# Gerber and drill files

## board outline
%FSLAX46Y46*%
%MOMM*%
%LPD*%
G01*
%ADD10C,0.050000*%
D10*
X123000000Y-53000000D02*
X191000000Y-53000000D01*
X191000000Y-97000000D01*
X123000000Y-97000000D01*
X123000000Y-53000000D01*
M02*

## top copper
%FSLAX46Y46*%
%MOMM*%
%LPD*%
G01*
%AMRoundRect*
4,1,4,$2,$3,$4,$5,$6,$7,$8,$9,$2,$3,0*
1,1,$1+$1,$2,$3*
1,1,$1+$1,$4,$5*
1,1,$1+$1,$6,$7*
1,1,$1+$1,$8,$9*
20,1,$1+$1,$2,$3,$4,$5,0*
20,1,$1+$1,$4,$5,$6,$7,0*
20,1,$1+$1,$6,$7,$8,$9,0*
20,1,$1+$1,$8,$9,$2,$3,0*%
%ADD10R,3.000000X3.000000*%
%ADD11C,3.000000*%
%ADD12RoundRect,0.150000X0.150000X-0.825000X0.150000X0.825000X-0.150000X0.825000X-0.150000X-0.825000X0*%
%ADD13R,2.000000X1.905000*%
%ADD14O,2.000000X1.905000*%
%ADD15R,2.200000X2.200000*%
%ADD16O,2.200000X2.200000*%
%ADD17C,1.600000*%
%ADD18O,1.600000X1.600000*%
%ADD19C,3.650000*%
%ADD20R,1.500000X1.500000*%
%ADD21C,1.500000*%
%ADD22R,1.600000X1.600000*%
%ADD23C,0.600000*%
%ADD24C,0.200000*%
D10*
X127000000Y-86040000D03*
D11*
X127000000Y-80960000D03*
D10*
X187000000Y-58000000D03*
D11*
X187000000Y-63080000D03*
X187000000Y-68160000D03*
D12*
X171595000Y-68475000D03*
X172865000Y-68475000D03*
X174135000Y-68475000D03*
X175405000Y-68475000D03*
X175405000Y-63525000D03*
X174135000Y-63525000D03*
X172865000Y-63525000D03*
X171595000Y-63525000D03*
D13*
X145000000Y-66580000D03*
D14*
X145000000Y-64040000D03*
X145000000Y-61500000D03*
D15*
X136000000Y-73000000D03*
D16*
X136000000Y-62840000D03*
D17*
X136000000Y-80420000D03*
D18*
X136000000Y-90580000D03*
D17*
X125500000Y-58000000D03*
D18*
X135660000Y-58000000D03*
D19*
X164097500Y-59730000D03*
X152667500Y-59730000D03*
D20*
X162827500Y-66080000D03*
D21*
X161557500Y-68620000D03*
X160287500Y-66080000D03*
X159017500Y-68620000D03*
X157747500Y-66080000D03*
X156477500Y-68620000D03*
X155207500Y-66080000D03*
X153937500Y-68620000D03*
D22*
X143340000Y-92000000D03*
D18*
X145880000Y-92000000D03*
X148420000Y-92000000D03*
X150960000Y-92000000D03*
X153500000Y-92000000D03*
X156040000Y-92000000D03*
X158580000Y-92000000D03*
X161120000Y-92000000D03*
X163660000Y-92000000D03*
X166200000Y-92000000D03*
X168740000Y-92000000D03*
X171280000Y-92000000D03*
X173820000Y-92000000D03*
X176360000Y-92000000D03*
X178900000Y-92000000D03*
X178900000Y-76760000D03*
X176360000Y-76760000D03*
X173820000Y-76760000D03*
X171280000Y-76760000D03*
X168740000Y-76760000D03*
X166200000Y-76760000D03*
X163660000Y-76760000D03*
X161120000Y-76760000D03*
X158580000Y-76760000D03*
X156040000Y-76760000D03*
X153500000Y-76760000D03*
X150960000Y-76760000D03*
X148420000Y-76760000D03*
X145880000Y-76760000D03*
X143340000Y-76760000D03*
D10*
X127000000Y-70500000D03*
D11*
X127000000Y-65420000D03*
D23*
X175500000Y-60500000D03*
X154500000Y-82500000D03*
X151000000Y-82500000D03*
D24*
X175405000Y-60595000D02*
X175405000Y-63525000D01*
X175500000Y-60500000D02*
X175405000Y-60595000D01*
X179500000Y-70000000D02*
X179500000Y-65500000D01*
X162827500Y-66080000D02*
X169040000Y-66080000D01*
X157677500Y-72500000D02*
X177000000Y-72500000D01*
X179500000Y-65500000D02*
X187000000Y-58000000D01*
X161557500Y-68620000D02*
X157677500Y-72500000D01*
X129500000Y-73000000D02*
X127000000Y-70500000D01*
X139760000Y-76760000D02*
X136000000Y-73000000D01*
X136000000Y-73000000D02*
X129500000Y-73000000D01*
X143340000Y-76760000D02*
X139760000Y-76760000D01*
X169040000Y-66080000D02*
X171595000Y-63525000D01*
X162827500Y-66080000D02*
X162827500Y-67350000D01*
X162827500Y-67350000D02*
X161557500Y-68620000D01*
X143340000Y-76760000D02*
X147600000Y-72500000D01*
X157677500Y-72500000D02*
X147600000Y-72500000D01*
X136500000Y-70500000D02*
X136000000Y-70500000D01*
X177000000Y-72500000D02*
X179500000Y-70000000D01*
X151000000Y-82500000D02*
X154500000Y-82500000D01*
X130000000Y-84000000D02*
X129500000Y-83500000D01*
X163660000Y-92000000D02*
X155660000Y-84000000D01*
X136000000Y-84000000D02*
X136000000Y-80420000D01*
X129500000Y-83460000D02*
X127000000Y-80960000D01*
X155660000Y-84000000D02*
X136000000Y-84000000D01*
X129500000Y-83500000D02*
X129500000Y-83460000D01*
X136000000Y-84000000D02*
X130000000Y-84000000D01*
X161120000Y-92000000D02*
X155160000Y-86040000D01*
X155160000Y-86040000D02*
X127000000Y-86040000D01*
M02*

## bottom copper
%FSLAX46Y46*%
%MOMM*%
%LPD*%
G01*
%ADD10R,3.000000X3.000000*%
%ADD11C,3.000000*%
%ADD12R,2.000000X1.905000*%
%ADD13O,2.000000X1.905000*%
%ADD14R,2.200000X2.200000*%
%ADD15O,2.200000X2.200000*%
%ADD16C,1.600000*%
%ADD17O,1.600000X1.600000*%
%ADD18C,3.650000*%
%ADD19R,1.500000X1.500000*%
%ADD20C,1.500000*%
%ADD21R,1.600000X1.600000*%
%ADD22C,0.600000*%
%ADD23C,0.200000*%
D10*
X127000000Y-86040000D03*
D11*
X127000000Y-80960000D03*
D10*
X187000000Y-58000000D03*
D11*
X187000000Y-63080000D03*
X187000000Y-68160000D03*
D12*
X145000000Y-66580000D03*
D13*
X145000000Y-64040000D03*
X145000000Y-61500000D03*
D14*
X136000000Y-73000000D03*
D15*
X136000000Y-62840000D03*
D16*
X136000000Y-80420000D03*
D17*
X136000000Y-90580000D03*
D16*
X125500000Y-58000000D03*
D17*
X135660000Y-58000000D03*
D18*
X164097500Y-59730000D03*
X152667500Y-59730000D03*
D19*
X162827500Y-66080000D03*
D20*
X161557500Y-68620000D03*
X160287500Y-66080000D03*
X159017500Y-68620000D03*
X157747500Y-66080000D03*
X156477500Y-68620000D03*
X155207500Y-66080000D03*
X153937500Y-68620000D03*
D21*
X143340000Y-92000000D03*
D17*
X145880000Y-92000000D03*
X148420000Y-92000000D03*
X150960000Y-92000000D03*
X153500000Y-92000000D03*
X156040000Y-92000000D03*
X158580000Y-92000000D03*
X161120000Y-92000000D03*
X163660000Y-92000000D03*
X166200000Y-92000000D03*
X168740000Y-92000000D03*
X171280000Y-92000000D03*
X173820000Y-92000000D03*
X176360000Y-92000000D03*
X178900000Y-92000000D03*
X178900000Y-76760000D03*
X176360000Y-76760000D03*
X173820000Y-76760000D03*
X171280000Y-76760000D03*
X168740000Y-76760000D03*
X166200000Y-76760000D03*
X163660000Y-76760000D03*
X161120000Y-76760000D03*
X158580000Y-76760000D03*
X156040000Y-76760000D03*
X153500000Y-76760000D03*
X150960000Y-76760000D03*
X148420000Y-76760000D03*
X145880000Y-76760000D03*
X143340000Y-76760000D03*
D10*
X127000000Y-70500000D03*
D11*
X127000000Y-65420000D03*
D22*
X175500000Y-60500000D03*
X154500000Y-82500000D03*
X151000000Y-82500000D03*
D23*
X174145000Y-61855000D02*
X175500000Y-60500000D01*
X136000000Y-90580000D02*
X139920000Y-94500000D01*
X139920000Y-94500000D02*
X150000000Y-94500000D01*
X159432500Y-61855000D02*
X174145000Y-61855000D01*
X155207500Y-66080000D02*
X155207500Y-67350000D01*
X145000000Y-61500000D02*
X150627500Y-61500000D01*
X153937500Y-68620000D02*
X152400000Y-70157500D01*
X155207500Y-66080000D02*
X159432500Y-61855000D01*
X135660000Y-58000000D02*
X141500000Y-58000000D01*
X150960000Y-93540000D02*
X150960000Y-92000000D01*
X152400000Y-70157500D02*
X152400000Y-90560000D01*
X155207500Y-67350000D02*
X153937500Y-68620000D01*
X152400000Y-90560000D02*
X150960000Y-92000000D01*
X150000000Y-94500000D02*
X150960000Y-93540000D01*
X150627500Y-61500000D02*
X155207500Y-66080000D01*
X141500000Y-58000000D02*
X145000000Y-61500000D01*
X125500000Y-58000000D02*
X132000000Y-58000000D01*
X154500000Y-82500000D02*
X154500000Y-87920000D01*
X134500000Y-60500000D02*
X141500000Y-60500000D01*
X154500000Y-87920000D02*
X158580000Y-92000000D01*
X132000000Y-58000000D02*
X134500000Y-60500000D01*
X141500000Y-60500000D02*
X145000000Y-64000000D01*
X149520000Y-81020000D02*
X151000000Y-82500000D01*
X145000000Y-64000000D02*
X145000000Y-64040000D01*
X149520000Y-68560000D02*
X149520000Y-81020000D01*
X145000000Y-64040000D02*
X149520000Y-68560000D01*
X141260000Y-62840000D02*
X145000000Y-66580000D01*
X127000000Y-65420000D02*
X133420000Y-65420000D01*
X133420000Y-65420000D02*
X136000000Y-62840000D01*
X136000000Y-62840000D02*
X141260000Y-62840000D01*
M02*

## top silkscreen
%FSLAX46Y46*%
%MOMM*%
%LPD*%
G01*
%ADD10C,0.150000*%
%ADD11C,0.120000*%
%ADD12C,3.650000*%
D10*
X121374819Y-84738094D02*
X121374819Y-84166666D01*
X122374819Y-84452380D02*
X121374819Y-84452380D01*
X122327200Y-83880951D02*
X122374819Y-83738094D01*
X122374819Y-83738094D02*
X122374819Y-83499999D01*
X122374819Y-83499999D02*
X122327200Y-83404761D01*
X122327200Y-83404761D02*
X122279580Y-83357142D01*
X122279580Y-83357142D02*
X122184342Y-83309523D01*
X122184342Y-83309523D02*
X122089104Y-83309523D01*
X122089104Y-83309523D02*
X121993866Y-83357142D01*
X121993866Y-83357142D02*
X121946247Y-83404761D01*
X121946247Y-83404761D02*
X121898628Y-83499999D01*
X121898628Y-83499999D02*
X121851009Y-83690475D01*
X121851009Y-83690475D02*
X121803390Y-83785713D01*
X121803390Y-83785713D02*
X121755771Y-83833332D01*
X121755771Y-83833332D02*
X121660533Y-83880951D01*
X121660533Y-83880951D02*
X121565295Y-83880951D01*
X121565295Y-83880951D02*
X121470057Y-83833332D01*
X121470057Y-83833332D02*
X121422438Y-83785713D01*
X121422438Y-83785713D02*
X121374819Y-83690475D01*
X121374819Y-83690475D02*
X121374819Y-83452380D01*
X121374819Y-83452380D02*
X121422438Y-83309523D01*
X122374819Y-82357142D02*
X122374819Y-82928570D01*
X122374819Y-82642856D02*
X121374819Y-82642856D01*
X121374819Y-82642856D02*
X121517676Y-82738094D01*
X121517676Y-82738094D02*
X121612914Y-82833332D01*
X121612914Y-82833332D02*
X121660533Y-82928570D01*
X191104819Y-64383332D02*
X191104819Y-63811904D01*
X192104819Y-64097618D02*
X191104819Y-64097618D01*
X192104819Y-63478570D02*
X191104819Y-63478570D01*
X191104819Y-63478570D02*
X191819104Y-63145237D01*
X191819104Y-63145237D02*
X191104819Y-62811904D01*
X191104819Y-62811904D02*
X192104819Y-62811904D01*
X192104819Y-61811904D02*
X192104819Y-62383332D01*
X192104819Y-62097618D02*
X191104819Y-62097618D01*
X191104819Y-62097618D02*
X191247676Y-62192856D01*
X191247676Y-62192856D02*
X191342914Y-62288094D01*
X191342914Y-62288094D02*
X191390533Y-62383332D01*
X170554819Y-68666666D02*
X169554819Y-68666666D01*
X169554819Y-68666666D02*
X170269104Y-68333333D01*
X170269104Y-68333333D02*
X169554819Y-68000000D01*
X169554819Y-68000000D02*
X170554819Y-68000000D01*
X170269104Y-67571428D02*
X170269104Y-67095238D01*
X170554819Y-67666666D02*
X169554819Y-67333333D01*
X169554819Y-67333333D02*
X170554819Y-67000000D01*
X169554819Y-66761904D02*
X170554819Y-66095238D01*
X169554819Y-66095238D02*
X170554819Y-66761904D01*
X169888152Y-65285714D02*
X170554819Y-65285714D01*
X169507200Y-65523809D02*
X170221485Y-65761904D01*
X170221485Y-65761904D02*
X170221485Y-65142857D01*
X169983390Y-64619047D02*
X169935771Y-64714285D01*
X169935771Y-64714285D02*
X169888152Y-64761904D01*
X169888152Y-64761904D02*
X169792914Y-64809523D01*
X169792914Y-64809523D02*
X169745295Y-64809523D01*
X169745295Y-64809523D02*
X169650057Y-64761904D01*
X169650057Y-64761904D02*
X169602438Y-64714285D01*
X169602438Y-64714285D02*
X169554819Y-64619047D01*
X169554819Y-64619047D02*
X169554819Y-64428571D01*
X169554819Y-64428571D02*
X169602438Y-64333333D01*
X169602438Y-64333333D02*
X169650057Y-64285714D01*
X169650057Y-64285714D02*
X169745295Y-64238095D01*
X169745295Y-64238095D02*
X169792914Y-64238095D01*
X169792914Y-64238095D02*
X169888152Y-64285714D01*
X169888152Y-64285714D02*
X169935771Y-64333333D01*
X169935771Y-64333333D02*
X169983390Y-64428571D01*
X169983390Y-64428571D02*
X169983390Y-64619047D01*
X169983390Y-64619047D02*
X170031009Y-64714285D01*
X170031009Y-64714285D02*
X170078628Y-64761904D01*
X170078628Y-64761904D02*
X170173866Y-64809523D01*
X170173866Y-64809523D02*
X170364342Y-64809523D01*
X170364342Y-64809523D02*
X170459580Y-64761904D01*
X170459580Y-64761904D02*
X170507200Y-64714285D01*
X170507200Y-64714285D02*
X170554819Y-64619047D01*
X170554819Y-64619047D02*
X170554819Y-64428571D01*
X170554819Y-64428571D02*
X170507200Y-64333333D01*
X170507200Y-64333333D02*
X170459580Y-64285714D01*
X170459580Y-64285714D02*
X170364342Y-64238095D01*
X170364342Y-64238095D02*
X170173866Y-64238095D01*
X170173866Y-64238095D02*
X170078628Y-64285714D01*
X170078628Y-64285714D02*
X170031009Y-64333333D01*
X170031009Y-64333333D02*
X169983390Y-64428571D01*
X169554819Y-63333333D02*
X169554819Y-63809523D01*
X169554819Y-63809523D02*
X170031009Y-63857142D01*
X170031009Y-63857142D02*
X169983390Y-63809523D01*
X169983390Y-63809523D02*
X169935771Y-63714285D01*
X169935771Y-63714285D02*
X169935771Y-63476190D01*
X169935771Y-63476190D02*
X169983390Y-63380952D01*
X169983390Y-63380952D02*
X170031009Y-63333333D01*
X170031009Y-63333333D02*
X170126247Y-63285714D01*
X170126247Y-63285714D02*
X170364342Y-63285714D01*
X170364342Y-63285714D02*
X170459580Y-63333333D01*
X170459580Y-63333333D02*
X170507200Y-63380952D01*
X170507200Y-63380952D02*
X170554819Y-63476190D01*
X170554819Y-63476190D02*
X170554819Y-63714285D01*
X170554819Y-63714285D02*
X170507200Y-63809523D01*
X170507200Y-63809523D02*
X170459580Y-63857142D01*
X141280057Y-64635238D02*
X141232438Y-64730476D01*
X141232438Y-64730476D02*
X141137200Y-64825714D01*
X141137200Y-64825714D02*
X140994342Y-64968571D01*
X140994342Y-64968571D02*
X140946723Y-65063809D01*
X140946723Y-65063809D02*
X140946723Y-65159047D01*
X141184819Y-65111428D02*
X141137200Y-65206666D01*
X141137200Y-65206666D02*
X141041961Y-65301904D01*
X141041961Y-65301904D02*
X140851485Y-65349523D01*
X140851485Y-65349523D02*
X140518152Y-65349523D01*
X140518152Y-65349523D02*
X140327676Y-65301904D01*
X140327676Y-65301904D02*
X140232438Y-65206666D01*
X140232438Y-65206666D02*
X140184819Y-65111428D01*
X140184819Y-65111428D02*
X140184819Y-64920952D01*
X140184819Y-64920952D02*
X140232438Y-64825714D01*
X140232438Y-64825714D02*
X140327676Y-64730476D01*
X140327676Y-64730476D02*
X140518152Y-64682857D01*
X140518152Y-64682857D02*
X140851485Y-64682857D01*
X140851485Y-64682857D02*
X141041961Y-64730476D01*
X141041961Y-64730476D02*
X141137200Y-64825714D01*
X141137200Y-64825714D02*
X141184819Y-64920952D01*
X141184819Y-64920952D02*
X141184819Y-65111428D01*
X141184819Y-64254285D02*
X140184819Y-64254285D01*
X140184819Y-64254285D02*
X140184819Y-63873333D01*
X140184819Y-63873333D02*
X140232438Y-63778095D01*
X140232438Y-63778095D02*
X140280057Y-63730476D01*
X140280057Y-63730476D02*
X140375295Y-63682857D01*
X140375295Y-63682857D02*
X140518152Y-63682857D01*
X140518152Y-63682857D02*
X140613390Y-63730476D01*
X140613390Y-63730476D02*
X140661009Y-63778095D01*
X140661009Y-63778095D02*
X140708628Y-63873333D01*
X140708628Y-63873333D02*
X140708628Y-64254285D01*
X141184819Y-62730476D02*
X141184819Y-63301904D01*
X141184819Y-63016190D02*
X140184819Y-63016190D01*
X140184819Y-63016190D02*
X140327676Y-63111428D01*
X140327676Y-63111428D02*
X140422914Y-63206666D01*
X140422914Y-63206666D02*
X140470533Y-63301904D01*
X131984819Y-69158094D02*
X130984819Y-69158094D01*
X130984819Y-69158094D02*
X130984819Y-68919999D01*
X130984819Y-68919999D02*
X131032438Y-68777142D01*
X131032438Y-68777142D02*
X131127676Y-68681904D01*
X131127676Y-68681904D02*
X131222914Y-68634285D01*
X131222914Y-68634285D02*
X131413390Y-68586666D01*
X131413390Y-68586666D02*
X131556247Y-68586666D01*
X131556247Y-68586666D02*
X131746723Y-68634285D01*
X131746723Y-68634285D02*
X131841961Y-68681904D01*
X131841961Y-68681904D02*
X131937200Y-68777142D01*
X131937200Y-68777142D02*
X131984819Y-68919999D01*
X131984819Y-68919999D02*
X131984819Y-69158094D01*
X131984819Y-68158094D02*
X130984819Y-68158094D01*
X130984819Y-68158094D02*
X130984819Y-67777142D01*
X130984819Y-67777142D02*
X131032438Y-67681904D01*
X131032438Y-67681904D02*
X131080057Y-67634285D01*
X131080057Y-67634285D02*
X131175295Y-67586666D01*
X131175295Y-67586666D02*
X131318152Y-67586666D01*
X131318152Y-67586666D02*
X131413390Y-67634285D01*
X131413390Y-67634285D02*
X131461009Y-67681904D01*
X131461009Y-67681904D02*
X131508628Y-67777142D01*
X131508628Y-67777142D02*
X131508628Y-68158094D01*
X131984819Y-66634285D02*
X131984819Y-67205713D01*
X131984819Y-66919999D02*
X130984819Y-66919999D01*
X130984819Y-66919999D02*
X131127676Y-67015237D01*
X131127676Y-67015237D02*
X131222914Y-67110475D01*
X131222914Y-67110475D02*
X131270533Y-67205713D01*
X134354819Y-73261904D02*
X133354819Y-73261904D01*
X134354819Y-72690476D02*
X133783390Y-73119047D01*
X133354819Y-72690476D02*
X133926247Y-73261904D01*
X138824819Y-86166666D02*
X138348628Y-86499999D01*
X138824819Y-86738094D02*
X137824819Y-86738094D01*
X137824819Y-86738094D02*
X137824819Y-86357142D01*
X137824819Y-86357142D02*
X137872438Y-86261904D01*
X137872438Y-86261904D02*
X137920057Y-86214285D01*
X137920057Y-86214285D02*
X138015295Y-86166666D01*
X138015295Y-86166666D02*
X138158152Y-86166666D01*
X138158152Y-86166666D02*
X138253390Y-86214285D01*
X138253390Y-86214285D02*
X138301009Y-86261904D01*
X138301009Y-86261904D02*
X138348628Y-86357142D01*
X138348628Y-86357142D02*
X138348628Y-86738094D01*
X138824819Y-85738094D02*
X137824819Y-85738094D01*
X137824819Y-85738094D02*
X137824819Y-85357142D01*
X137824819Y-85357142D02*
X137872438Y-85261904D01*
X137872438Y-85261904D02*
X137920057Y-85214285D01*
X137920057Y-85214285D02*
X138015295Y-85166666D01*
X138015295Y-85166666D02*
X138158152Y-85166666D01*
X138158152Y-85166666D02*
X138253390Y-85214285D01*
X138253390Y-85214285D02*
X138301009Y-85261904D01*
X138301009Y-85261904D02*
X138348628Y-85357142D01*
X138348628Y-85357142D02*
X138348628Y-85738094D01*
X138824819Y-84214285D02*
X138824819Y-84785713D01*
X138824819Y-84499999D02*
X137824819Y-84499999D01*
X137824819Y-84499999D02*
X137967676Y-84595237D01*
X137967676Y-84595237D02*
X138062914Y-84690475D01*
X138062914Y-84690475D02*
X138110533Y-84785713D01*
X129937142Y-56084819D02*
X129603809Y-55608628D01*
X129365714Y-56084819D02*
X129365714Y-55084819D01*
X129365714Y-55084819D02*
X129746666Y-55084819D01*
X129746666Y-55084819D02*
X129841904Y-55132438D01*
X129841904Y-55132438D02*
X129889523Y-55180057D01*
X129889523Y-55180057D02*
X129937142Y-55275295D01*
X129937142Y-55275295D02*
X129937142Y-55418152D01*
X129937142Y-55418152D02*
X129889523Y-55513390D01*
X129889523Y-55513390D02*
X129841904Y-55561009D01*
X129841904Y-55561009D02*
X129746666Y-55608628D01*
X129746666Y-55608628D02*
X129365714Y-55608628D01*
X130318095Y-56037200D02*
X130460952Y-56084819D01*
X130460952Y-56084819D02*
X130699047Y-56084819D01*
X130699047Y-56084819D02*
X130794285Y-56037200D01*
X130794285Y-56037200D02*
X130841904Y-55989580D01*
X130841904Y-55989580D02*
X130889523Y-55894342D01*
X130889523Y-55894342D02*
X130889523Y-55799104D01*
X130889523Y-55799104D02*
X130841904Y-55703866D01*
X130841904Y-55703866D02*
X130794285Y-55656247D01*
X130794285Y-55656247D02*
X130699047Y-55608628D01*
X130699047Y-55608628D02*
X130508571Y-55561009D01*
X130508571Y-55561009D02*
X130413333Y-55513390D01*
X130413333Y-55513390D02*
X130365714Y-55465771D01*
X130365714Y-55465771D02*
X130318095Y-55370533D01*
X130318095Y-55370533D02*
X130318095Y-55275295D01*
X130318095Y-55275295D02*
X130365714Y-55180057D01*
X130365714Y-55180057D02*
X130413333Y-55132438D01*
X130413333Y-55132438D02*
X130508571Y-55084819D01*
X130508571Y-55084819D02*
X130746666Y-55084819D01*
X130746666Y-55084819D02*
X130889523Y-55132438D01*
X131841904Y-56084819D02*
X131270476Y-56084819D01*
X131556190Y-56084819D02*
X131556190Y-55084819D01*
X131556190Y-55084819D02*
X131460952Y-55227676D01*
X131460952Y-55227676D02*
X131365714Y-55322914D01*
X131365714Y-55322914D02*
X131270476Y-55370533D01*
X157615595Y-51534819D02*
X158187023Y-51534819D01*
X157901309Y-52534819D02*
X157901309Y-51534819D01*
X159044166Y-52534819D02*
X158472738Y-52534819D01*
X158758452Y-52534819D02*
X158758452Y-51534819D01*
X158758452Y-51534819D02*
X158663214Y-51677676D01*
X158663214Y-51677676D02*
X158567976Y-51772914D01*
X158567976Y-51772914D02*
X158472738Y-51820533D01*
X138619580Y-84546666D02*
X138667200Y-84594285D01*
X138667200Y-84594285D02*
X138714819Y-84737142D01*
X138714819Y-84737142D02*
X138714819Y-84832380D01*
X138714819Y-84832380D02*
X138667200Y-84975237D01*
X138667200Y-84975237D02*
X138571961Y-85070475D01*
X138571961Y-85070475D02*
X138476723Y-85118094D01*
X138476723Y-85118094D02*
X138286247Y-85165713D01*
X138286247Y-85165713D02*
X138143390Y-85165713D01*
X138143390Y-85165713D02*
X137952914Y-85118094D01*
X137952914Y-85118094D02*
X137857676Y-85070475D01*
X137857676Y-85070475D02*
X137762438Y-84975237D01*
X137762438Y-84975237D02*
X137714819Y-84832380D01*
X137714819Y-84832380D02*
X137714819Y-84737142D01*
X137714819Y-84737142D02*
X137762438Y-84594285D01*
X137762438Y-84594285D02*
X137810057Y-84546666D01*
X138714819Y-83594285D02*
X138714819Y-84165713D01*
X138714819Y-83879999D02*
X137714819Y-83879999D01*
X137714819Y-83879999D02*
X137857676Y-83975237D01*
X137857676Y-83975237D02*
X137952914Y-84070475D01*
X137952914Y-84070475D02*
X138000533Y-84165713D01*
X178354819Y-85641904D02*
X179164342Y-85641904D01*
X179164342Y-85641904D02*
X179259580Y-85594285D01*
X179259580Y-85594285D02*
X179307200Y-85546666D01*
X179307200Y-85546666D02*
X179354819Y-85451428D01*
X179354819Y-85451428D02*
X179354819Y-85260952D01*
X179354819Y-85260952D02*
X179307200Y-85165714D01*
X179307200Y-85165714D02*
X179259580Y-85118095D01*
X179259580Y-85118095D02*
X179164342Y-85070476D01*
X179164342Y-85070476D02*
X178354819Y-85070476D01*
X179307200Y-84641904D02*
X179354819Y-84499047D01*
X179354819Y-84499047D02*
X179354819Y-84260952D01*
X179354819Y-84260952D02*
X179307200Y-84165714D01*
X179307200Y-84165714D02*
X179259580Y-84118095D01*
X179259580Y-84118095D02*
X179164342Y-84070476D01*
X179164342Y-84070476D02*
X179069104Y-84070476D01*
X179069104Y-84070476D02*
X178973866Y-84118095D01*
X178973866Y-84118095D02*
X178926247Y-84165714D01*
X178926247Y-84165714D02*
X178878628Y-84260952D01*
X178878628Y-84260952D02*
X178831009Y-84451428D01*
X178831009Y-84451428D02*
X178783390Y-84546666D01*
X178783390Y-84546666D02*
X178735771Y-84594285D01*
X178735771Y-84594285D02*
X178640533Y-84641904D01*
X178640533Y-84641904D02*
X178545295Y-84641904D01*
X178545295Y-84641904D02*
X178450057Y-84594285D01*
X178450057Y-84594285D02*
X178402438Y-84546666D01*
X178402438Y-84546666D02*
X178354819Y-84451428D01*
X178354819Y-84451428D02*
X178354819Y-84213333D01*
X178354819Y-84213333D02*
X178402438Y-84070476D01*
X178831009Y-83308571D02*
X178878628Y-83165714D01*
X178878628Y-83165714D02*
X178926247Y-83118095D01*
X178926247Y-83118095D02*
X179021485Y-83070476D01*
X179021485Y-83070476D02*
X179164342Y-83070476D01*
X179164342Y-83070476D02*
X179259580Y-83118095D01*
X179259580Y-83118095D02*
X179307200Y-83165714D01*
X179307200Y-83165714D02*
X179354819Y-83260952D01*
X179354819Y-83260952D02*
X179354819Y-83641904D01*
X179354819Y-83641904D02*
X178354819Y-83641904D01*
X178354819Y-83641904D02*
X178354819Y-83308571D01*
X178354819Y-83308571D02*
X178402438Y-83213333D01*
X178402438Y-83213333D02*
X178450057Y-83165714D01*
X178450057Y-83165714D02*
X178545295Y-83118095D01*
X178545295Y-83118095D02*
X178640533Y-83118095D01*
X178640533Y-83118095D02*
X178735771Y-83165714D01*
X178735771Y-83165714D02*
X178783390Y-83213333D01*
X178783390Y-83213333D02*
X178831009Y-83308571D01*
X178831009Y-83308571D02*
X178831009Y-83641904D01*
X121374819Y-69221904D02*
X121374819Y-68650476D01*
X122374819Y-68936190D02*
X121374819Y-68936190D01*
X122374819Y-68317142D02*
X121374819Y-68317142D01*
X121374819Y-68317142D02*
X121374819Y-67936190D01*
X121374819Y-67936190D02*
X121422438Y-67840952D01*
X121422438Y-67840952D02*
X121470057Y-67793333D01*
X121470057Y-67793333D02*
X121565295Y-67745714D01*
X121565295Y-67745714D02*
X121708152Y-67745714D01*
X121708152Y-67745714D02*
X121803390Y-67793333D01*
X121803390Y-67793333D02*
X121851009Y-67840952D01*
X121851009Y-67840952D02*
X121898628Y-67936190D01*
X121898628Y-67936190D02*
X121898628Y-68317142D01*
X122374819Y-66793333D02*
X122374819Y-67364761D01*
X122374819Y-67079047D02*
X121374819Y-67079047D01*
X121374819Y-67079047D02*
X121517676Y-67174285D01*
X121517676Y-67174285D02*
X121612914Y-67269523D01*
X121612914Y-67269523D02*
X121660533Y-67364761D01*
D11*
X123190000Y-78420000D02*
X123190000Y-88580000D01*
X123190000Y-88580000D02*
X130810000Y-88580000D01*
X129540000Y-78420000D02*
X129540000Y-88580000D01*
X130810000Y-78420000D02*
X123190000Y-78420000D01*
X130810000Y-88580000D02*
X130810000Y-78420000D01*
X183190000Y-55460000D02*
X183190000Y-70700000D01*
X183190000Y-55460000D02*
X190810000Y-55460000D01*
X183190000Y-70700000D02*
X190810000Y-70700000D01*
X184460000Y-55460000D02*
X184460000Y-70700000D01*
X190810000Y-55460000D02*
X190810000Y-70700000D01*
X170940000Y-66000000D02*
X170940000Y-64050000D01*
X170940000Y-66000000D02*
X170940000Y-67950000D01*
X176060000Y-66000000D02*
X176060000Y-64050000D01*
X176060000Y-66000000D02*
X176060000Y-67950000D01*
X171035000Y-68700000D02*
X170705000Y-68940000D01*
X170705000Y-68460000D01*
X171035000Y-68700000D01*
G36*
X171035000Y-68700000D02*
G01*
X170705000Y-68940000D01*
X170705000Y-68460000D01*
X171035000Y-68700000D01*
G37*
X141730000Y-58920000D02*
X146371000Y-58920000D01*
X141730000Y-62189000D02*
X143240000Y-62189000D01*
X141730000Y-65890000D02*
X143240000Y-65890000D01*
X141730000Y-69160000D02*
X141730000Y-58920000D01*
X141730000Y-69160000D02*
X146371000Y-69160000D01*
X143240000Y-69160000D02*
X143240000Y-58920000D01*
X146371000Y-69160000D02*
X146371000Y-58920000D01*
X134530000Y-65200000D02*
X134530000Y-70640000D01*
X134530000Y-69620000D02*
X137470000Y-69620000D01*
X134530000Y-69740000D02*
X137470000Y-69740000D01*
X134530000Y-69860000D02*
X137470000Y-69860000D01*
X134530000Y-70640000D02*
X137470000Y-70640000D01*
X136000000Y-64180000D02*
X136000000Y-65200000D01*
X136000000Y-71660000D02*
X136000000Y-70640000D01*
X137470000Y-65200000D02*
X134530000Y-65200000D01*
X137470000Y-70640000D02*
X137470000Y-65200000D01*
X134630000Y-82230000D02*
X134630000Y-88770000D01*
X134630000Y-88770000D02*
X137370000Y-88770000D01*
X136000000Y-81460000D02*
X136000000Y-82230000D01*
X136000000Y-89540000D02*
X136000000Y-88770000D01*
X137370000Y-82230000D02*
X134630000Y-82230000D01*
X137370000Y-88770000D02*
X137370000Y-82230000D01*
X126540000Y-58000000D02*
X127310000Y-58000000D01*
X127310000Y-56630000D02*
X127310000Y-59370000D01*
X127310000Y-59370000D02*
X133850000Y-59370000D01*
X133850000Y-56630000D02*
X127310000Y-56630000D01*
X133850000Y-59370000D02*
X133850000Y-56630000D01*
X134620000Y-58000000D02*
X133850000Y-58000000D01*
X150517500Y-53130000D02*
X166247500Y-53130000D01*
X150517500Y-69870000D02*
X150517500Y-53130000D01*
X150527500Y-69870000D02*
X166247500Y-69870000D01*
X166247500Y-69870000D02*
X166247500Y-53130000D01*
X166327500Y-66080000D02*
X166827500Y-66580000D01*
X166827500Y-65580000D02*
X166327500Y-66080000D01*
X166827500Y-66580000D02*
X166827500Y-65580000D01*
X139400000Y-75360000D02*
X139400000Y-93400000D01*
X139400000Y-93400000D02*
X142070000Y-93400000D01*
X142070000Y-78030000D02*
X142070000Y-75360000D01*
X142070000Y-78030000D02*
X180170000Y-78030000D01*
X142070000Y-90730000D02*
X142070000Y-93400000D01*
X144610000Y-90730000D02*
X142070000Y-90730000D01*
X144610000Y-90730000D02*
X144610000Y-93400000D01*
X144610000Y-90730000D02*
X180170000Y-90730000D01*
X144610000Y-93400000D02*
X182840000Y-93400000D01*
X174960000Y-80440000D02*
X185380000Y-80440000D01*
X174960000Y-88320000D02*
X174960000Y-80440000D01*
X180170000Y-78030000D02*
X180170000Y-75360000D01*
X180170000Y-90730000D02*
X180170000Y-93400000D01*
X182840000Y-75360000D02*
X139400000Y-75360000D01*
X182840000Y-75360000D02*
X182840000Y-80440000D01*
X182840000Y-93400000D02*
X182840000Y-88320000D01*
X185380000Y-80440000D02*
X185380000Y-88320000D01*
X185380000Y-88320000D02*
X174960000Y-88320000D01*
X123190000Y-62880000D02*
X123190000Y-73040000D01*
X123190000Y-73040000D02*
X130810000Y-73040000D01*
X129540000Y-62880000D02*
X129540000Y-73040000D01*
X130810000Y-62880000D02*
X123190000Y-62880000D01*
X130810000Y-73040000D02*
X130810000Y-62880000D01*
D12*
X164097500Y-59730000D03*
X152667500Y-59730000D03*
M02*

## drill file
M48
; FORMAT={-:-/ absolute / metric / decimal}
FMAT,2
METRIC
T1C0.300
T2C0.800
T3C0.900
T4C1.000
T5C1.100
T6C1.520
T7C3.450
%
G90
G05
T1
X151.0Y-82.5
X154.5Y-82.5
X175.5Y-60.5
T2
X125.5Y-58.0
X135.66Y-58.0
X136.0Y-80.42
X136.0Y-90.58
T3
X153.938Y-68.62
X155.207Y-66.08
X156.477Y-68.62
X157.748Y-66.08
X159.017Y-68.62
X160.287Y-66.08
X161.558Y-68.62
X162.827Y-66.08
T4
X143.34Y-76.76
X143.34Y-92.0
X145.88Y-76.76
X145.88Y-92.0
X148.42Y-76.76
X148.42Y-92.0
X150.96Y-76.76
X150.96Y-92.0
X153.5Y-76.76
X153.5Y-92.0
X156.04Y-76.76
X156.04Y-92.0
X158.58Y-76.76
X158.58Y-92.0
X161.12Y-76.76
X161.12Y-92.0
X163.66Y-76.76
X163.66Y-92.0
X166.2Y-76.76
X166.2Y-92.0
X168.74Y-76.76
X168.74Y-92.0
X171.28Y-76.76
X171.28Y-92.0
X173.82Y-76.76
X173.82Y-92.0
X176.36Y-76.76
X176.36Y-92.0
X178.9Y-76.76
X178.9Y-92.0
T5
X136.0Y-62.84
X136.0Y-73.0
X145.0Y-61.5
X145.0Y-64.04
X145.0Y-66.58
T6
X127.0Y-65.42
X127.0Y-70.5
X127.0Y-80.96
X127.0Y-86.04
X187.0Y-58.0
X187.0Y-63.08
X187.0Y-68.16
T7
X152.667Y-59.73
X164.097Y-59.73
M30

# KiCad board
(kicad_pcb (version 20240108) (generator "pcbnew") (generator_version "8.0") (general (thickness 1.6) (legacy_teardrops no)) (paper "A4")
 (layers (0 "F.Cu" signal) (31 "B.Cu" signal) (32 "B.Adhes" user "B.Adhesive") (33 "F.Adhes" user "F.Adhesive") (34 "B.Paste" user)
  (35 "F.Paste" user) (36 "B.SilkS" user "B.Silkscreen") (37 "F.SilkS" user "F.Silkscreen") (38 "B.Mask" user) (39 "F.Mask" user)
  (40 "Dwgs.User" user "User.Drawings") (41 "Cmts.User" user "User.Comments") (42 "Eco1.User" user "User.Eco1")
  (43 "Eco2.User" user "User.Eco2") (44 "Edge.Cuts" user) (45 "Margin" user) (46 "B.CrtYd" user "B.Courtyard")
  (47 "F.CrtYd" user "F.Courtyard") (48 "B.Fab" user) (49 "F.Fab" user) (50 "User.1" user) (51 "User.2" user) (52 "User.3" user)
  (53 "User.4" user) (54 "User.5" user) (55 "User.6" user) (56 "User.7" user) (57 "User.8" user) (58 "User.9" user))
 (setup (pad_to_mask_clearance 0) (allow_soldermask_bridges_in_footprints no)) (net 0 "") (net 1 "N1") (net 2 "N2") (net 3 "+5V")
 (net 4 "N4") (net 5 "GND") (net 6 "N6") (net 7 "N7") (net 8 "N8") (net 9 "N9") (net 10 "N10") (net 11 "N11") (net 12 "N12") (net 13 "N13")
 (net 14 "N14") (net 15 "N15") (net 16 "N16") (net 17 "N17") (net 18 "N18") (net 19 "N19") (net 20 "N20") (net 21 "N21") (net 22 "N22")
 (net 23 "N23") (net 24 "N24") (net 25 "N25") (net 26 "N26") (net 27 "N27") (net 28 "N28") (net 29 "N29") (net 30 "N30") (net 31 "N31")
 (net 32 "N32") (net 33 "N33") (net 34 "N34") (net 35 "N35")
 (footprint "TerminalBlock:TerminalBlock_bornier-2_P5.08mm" (layer "F.Cu") (at 127 86.04 90)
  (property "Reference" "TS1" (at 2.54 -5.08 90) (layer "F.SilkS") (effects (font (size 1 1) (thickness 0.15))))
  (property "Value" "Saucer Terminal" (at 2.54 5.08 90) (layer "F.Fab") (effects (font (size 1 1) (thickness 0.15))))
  (fp_line (start 7.62 -3.81) (end -2.54 -3.81) (stroke (width 0.12) (type solid)) (layer "F.SilkS"))
  (fp_line (start -2.54 -3.81) (end -2.54 3.81) (stroke (width 0.12) (type solid)) (layer "F.SilkS"))
  (fp_line (start 7.62 2.54) (end -2.54 2.54) (stroke (width 0.12) (type solid)) (layer "F.SilkS"))
  (fp_line (start 7.62 3.81) (end 7.62 -3.81) (stroke (width 0.12) (type solid)) (layer "F.SilkS"))
  (fp_line (start -2.54 3.81) (end 7.62 3.81) (stroke (width 0.12) (type solid)) (layer "F.SilkS"))
  (pad "1" thru_hole rect (at 0 0 90) (size 3 3) (drill 1.52) (layers "*.Cu" "*.Mask") (remove_unused_layers no) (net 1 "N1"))
  (pad "2" thru_hole circle (at 5.08 0 90) (size 3 3) (drill 1.52) (layers "*.Cu" "*.Mask") (remove_unused_layers no) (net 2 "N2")))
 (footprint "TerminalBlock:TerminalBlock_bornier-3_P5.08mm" (layer "F.Cu") (at 187 58 -90)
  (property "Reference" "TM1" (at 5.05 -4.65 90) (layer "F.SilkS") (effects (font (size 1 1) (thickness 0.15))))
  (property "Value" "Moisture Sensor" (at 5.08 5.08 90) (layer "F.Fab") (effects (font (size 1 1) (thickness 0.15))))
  (fp_line (start -2.54 3.81) (end 12.7 3.81) (stroke (width 0.12) (type solid)) (layer "F.SilkS"))
  (fp_line (start -2.54 3.81) (end -2.54 -3.81) (stroke (width 0.12) (type solid)) (layer "F.SilkS"))
  (fp_line (start 12.7 3.81) (end 12.7 -3.81) (stroke (width 0.12) (type solid)) (layer "F.SilkS"))
  (fp_line (start -2.54 2.54) (end 12.7 2.54) (stroke (width 0.12) (type solid)) (layer "F.SilkS"))
  (fp_line (start -2.54 -3.81) (end 12.7 -3.81) (stroke (width 0.12) (type solid)) (layer "F.SilkS"))
  (pad "1" thru_hole rect (at 0 0 270) (size 3 3) (drill 1.52) (layers "*.Cu" "*.Mask") (remove_unused_layers no) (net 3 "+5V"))
  (pad "2" thru_hole circle (at 5.08 0 270) (size 3 3) (drill 1.52) (layers "*.Cu" "*.Mask") (remove_unused_layers no) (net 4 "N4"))
  (pad "3" thru_hole circle (at 10.16 0 270) (size 3 3) (drill 1.52) (layers "*.Cu" "*.Mask") (remove_unused_layers no) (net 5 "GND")))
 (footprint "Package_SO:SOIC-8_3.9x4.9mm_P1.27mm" (layer "F.Cu") (at 173.5 66 90)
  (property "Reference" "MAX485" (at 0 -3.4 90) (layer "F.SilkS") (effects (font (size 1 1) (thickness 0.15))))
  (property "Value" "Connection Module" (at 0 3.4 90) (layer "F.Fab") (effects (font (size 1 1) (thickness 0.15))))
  (fp_line (start 0 -2.56) (end 1.95 -2.56) (stroke (width 0.12) (type solid)) (layer "F.SilkS"))
  (fp_line (start 0 -2.56) (end -1.95 -2.56) (stroke (width 0.12) (type solid)) (layer "F.SilkS"))
  (fp_line (start 0 2.56) (end 1.95 2.56) (stroke (width 0.12) (type solid)) (layer "F.SilkS"))
  (fp_line (start 0 2.56) (end -1.95 2.56) (stroke (width 0.12) (type solid)) (layer "F.SilkS"))
  (fp_poly
   (pts (xy -2.7 -2.465) (xy -2.94 -2.795) (xy -2.46 -2.795) (xy -2.7 -2.465)) (stroke (width 0.12) (type solid)) (fill solid)
   (layer "F.SilkS"))
  (pad "1" smd roundrect (at -2.475 -1.905 90) (size 1.95 0.6) (layers "F.Cu" "F.Paste" "F.Mask") (roundrect_rratio 0.25) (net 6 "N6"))
  (pad "2" smd roundrect (at -2.475 -0.635 90) (size 1.95 0.6) (layers "F.Cu" "F.Paste" "F.Mask") (roundrect_rratio 0.25) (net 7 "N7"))
  (pad "3" smd roundrect (at -2.475 0.635 90) (size 1.95 0.6) (layers "F.Cu" "F.Paste" "F.Mask") (roundrect_rratio 0.25) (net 7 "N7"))
  (pad "4" smd roundrect (at -2.475 1.905 90) (size 1.95 0.6) (layers "F.Cu" "F.Paste" "F.Mask") (roundrect_rratio 0.25) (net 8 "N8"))
  (pad "5" smd roundrect (at 2.475 1.905 90) (size 1.95 0.6) (layers "F.Cu" "F.Paste" "F.Mask") (roundrect_rratio 0.25) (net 5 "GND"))
  (pad "6" smd roundrect (at 2.475 0.635 90) (size 1.95 0.6) (layers "F.Cu" "F.Paste" "F.Mask") (roundrect_rratio 0.25) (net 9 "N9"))
  (pad "7" smd roundrect (at 2.475 -0.635 90) (size 1.95 0.6) (layers "F.Cu" "F.Paste" "F.Mask") (roundrect_rratio 0.25) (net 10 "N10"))
  (pad "8" smd roundrect (at 2.475 -1.905 90) (size 1.95 0.6) (layers "F.Cu" "F.Paste" "F.Mask") (roundrect_rratio 0.25) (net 3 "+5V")))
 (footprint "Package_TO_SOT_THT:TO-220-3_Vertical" (layer "F.Cu") (at 145 66.58 90)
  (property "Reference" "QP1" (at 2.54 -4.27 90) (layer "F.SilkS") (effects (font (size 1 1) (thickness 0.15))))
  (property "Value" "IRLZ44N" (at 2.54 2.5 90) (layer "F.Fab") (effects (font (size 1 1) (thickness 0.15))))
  (fp_line (start 7.66 -3.27) (end 7.66 1.371) (stroke (width 0.12) (type solid)) (layer "F.SilkS"))
  (fp_line (start 4.391 -3.27) (end 4.391 -1.76) (stroke (width 0.12) (type solid)) (layer "F.SilkS"))
  (fp_line (start 0.69 -3.27) (end 0.69 -1.76) (stroke (width 0.12) (type solid)) (layer "F.SilkS"))
  (fp_line (start -2.58 -3.27) (end 7.66 -3.27) (stroke (width 0.12) (type solid)) (layer "F.SilkS"))
  (fp_line (start -2.58 -3.27) (end -2.58 1.371) (stroke (width 0.12) (type solid)) (layer "F.SilkS"))
  (fp_line (start -2.58 -1.76) (end 7.66 -1.76) (stroke (width 0.12) (type solid)) (layer "F.SilkS"))
  (fp_line (start -2.58 1.371) (end 7.66 1.371) (stroke (width 0.12) (type solid)) (layer "F.SilkS"))
  (pad "1" thru_hole rect (at 0 0 90) (size 1.905 2) (drill 1.1) (layers "*.Cu" "*.Mask") (remove_unused_layers no) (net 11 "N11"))
  (pad "2" thru_hole oval (at 2.54 0 90) (size 1.905 2) (drill 1.1) (layers "*.Cu" "*.Mask") (remove_unused_layers no) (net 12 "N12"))
  (pad "3" thru_hole oval (at 5.08 0 90) (size 1.905 2) (drill 1.1) (layers "*.Cu" "*.Mask") (remove_unused_layers no) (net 5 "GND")))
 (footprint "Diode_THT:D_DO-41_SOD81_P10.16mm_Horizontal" (layer "F.Cu") (at 136 73 90)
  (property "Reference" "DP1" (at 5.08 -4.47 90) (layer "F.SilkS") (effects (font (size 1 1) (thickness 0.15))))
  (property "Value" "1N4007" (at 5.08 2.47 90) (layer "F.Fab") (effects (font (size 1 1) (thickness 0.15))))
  (fp_line (start 7.8 -1.47) (end 2.36 -1.47) (stroke (width 0.12) (type solid)) (layer "F.SilkS"))
  (fp_line (start 3.38 -1.47) (end 3.38 1.47) (stroke (width 0.12) (type solid)) (layer "F.SilkS"))
  (fp_line (start 3.26 -1.47) (end 3.26 1.47) (stroke (width 0.12) (type solid)) (layer "F.SilkS"))
  (fp_line (start 3.14 -1.47) (end 3.14 1.47) (stroke (width 0.12) (type solid)) (layer "F.SilkS"))
  (fp_line (start 2.36 -1.47) (end 2.36 1.47) (stroke (width 0.12) (type solid)) (layer "F.SilkS"))
  (fp_line (start 8.82 0) (end 7.8 0) (stroke (width 0.12) (type solid)) (layer "F.SilkS"))
  (fp_line (start 1.34 0) (end 2.36 0) (stroke (width 0.12) (type solid)) (layer "F.SilkS"))
  (fp_line (start 7.8 1.47) (end 7.8 -1.47) (stroke (width 0.12) (type solid)) (layer "F.SilkS"))
  (fp_line (start 2.36 1.47) (end 7.8 1.47) (stroke (width 0.12) (type solid)) (layer "F.SilkS"))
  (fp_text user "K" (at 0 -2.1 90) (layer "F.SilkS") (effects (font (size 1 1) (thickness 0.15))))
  (pad "1" thru_hole rect (at 0 0 90) (size 2.2 2.2) (drill 1.1) (layers "*.Cu" "*.Mask") (remove_unused_layers no) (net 3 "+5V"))
  (pad "2" thru_hole oval (at 10.16 0 90) (size 2.2 2.2) (drill 1.1) (layers "*.Cu" "*.Mask") (remove_unused_layers no) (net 11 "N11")))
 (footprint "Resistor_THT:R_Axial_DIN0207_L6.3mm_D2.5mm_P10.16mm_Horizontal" (layer "F.Cu") (at 136 80.42 -90)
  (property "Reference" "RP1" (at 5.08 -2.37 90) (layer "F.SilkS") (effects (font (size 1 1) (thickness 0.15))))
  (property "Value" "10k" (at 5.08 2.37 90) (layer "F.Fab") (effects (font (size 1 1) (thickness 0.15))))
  (fp_line (start 1.81 1.37) (end 8.35 1.37) (stroke (width 0.12) (type solid)) (layer "F.SilkS"))
  (fp_line (start 8.35 1.37) (end 8.35 -1.37) (stroke (width 0.12) (type solid)) (layer "F.SilkS"))
  (fp_line (start 1.04 0) (end 1.81 0) (stroke (width 0.12) (type solid)) (layer "F.SilkS"))
  (fp_line (start 9.12 0) (end 8.35 0) (stroke (width 0.12) (type solid)) (layer "F.SilkS"))
  (fp_line (start 1.81 -1.37) (end 1.81 1.37) (stroke (width 0.12) (type solid)) (layer "F.SilkS"))
  (fp_line (start 8.35 -1.37) (end 1.81 -1.37) (stroke (width 0.12) (type solid)) (layer "F.SilkS"))
  (pad "1" thru_hole circle (at 0 0 270) (size 1.6 1.6) (drill 0.8) (layers "*.Cu" "*.Mask") (remove_unused_layers no) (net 2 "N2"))
  (pad "2" thru_hole oval (at 10.16 0 270) (size 1.6 1.6) (drill 0.8) (layers "*.Cu" "*.Mask") (remove_unused_layers no) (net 5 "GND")))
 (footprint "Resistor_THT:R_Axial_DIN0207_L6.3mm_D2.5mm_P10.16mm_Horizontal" (layer "F.Cu") (at 125.5 58)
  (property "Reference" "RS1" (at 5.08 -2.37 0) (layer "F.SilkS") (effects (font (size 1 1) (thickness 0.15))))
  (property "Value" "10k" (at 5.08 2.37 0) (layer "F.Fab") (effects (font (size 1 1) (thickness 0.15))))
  (fp_line (start 1.04 0) (end 1.81 0) (stroke (width 0.12) (type solid)) (layer "F.SilkS"))
  (fp_line (start 1.81 -1.37) (end 1.81 1.37) (stroke (width 0.12) (type solid)) (layer "F.SilkS"))
  (fp_line (start 1.81 1.37) (end 8.35 1.37) (stroke (width 0.12) (type solid)) (layer "F.SilkS"))
  (fp_line (start 8.35 -1.37) (end 1.81 -1.37) (stroke (width 0.12) (type solid)) (layer "F.SilkS"))
  (fp_line (start 8.35 1.37) (end 8.35 -1.37) (stroke (width 0.12) (type solid)) (layer "F.SilkS"))
  (fp_line (start 9.12 0) (end 8.35 0) (stroke (width 0.12) (type solid)) (layer "F.SilkS"))
  (pad "1" thru_hole circle (at 0 0) (size 1.6 1.6) (drill 0.8) (layers "*.Cu" "*.Mask") (remove_unused_layers no) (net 12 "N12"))
  (pad "2" thru_hole oval (at 10.16 0) (size 1.6 1.6) (drill 0.8) (layers "*.Cu" "*.Mask") (remove_unused_layers no) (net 5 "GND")))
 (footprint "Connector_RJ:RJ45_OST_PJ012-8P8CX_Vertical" (layer "F.Cu") (at 162.8275 66.08 180)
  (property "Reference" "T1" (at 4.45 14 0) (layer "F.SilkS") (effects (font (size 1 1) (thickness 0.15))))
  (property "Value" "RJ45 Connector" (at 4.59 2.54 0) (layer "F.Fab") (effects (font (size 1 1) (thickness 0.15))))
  (fp_line (start 12.31 12.95) (end -3.42 12.95) (stroke (width 0.12) (type solid)) (layer "F.SilkS"))
  (fp_line (start 12.31 -3.79) (end 12.31 12.95) (stroke (width 0.12) (type solid)) (layer "F.SilkS"))
  (fp_line (start 12.3 -3.79) (end -3.42 -3.79) (stroke (width 0.12) (type solid)) (layer "F.SilkS"))
  (fp_line (start -3.42 -3.79) (end -3.42 12.95) (stroke (width 0.12) (type solid)) (layer "F.SilkS"))
  (fp_line (start -3.5 0) (end -4 -0.5) (stroke (width 0.12) (type solid)) (layer "F.SilkS"))
  (fp_line (start -4 0.5) (end -3.5 0) (stroke (width 0.12) (type solid)) (layer "F.SilkS"))
  (fp_line (start -4 -0.5) (end -4 0.5) (stroke (width 0.12) (type solid)) (layer "F.SilkS"))
  (pad "" np_thru_hole circle (at -1.27 6.35 180) (size 3.65 3.65) (drill 3.45) (layers "*.Cu" "*.SilkS" "*.Mask"))
  (pad "" np_thru_hole circle (at 10.16 6.35 180) (size 3.65 3.65) (drill 3.45) (layers "*.Cu" "*.SilkS" "*.Mask"))
  (pad "1" thru_hole rect (at 0 0 180) (size 1.5 1.5) (drill 0.9) (layers "*.Cu" "*.Mask") (remove_unused_layers no) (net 3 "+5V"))
  (pad "2" thru_hole circle (at 1.27 -2.54 180) (size 1.5 1.5) (drill 0.9) (layers "*.Cu" "*.Mask") (remove_unused_layers no) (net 3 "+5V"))
  (pad "3" thru_hole circle (at 2.54 0 180) (size 1.5 1.5) (drill 0.9) (layers "*.Cu" "*.Mask") (remove_unused_layers no) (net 9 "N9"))
  (pad "4" thru_hole circle (at 3.81 -2.54 180) (size 1.5 1.5) (drill 0.9) (layers "*.Cu" "*.Mask") (remove_unused_layers no) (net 10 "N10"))
  (pad "5" thru_hole circle (at 5.08 0 180) (size 1.5 1.5) (drill 0.9) (layers "*.Cu" "*.Mask") (remove_unused_layers no) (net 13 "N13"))
  (pad "6" thru_hole circle (at 6.35 -2.54 180) (size 1.5 1.5) (drill 0.9) (layers "*.Cu" "*.Mask") (remove_unused_layers no) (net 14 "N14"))
  (pad "7" thru_hole circle (at 7.62 0 180) (size 1.5 1.5) (drill 0.9) (layers "*.Cu" "*.Mask") (remove_unused_layers no) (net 5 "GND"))
  (pad "8" thru_hole circle (at 8.89 -2.54 180) (size 1.5 1.5) (drill 0.9) (layers "*.Cu" "*.Mask") (remove_unused_layers no) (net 5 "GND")))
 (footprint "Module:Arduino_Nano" (layer "F.Cu") (at 143.34 92 90)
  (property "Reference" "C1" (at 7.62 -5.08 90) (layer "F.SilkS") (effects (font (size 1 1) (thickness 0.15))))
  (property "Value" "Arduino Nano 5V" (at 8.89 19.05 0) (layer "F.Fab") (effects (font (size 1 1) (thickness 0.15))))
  (fp_line (start 16.64 -3.94) (end -1.4 -3.94) (stroke (width 0.12) (type solid)) (layer "F.SilkS"))
  (fp_line (start -1.4 -3.94) (end -1.4 -1.27) (stroke (width 0.12) (type solid)) (layer "F.SilkS"))
  (fp_line (start 13.97 -1.27) (end 16.64 -1.27) (stroke (width 0.12) (type solid)) (layer "F.SilkS"))
  (fp_line (start 13.97 -1.27) (end 13.97 36.83) (stroke (width 0.12) (type solid)) (layer "F.SilkS"))
  (fp_line (start 1.27 -1.27) (end -1.4 -1.27) (stroke (width 0.12) (type solid)) (layer "F.SilkS"))
  (fp_line (start 1.27 1.27) (end 1.27 -1.27) (stroke (width 0.12) (type solid)) (layer "F.SilkS"))
  (fp_line (start 1.27 1.27) (end -1.4 1.27) (stroke (width 0.12) (type solid)) (layer "F.SilkS"))
  (fp_line (start 1.27 1.27) (end 1.27 36.83) (stroke (width 0.12) (type solid)) (layer "F.SilkS"))
  (fp_line (start -1.4 1.27) (end -1.4 39.5) (stroke (width 0.12) (type solid)) (layer "F.SilkS"))
  (fp_line (start 11.56 31.62) (end 11.56 42.04) (stroke (width 0.12) (type solid)) (layer "F.SilkS"))
  (fp_line (start 3.68 31.62) (end 11.56 31.62) (stroke (width 0.12) (type solid)) (layer "F.SilkS"))
  (fp_line (start 13.97 36.83) (end 16.64 36.83) (stroke (width 0.12) (type solid)) (layer "F.SilkS"))
  (fp_line (start 1.27 36.83) (end -1.4 36.83) (stroke (width 0.12) (type solid)) (layer "F.SilkS"))
  (fp_line (start 16.64 39.5) (end 16.64 -3.94) (stroke (width 0.12) (type solid)) (layer "F.SilkS"))
  (fp_line (start 16.64 39.5) (end 11.56 39.5) (stroke (width 0.12) (type solid)) (layer "F.SilkS"))
  (fp_line (start -1.4 39.5) (end 3.68 39.5) (stroke (width 0.12) (type solid)) (layer "F.SilkS"))
  (fp_line (start 11.56 42.04) (end 3.68 42.04) (stroke (width 0.12) (type solid)) (layer "F.SilkS"))
  (fp_line (start 3.68 42.04) (end 3.68 31.62) (stroke (width 0.12) (type solid)) (layer "F.SilkS"))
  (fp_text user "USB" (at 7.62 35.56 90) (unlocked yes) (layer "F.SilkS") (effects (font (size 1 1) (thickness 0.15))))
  (pad "1" thru_hole rect (at 0 0 90) (size 1.6 1.6) (drill 1) (layers "*.Cu" "*.Mask") (remove_unused_layers no) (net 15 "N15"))
  (pad "2" thru_hole oval (at 0 2.54 90) (size 1.6 1.6) (drill 1) (layers "*.Cu" "*.Mask") (remove_unused_layers no) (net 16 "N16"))
  (pad "3" thru_hole oval (at 0 5.08 90) (size 1.6 1.6) (drill 1) (layers "*.Cu" "*.Mask") (remove_unused_layers no) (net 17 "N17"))
  (pad "4" thru_hole oval (at 0 7.62 90) (size 1.6 1.6) (drill 1) (layers "*.Cu" "*.Mask") (remove_unused_layers no) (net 5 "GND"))
  (pad "5" thru_hole oval (at 0 10.16 90) (size 1.6 1.6) (drill 1) (layers "*.Cu" "*.Mask") (remove_unused_layers no) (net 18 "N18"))
  (pad "6" thru_hole oval (at 0 12.7 90) (size 1.6 1.6) (drill 1) (layers "*.Cu" "*.Mask") (remove_unused_layers no) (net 7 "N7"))
  (pad "7" thru_hole oval (at 0 15.24 90) (size 1.6 1.6) (drill 1) (layers "*.Cu" "*.Mask") (remove_unused_layers no) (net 12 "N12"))
  (pad "8" thru_hole oval (at 0 17.78 90) (size 1.6 1.6) (drill 1) (layers "*.Cu" "*.Mask") (remove_unused_layers no) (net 1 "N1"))
  (pad "9" thru_hole oval (at 0 20.32 90) (size 1.6 1.6) (drill 1) (layers "*.Cu" "*.Mask") (remove_unused_layers no) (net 2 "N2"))
  (pad "10" thru_hole oval (at 0 22.86 90) (size 1.6 1.6) (drill 1) (layers "*.Cu" "*.Mask") (remove_unused_layers no) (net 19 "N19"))
  (pad "11" thru_hole oval (at 0 25.4 90) (size 1.6 1.6) (drill 1) (layers "*.Cu" "*.Mask") (remove_unused_layers no) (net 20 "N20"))
  (pad "12" thru_hole oval (at 0 27.94 90) (size 1.6 1.6) (drill 1) (layers "*.Cu" "*.Mask") (remove_unused_layers no) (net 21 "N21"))
  (pad "13" thru_hole oval (at 0 30.48 90) (size 1.6 1.6) (drill 1) (layers "*.Cu" "*.Mask") (remove_unused_layers no) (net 6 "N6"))
  (pad "14" thru_hole oval (at 0 33.02 90) (size 1.6 1.6) (drill 1) (layers "*.Cu" "*.Mask") (remove_unused_layers no) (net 8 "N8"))
  (pad "15" thru_hole oval (at 0 35.56 90) (size 1.6 1.6) (drill 1) (layers "*.Cu" "*.Mask") (remove_unused_layers no) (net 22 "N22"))
  (pad "16" thru_hole oval (at 15.24 35.56 90) (size 1.6 1.6) (drill 1) (layers "*.Cu" "*.Mask") (remove_unused_layers no) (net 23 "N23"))
  (pad "17" thru_hole oval (at 15.24 33.02 90) (size 1.6 1.6) (drill 1) (layers "*.Cu" "*.Mask") (remove_unused_layers no) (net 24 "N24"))
  (pad "18" thru_hole oval (at 15.24 30.48 90) (size 1.6 1.6) (drill 1) (layers "*.Cu" "*.Mask") (remove_unused_layers no) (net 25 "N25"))
  (pad "19" thru_hole oval (at 15.24 27.94 90) (size 1.6 1.6) (drill 1) (layers "*.Cu" "*.Mask") (remove_unused_layers no) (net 4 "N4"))
  (pad "20" thru_hole oval (at 15.24 25.4 90) (size 1.6 1.6) (drill 1) (layers "*.Cu" "*.Mask") (remove_unused_layers no) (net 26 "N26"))
  (pad "21" thru_hole oval (at 15.24 22.86 90) (size 1.6 1.6) (drill 1) (layers "*.Cu" "*.Mask") (remove_unused_layers no) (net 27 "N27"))
  (pad "22" thru_hole oval (at 15.24 20.32 90) (size 1.6 1.6) (drill 1) (layers "*.Cu" "*.Mask") (remove_unused_layers no) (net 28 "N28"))
  (pad "23" thru_hole oval (at 15.24 17.78 90) (size 1.6 1.6) (drill 1) (layers "*.Cu" "*.Mask") (remove_unused_layers no) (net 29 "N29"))
  (pad "24" thru_hole oval (at 15.24 15.24 90) (size 1.6 1.6) (drill 1) (layers "*.Cu" "*.Mask") (remove_unused_layers no) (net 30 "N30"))
  (pad "25" thru_hole oval (at 15.24 12.7 90) (size 1.6 1.6) (drill 1) (layers "*.Cu" "*.Mask") (remove_unused_layers no) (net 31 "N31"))
  (pad "26" thru_hole oval (at 15.24 10.16 90) (size 1.6 1.6) (drill 1) (layers "*.Cu" "*.Mask") (remove_unused_layers no) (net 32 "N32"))
  (pad "27" thru_hole oval (at 15.24 7.62 90) (size 1.6 1.6) (drill 1) (layers "*.Cu" "*.Mask") (remove_unused_layers no) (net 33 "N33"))
  (pad "28" thru_hole oval (at 15.24 5.08 90) (size 1.6 1.6) (drill 1) (layers "*.Cu" "*.Mask") (remove_unused_layers no) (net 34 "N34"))
  (pad "29" thru_hole oval (at 15.24 2.54 90) (size 1.6 1.6) (drill 1) (layers "*.Cu" "*.Mask") (remove_unused_layers no) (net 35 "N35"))
  (pad "30" thru_hole oval (at 15.24 0 90) (size 1.6 1.6) (drill 1) (layers "*.Cu" "*.Mask") (remove_unused_layers no) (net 3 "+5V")))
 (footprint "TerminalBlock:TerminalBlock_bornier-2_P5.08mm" (layer "F.Cu") (at 127 70.5 90)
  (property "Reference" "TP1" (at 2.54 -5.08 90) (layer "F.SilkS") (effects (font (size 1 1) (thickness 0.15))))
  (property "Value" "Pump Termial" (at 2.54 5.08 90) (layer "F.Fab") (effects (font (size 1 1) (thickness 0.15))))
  (fp_line (start 7.62 -3.81) (end -2.54 -3.81) (stroke (width 0.12) (type solid)) (layer "F.SilkS"))
  (fp_line (start -2.54 -3.81) (end -2.54 3.81) (stroke (width 0.12) (type solid)) (layer "F.SilkS"))
  (fp_line (start 7.62 2.54) (end -2.54 2.54) (stroke (width 0.12) (type solid)) (layer "F.SilkS"))
  (fp_line (start 7.62 3.81) (end 7.62 -3.81) (stroke (width 0.12) (type solid)) (layer "F.SilkS"))
  (fp_line (start -2.54 3.81) (end 7.62 3.81) (stroke (width 0.12) (type solid)) (layer "F.SilkS"))
  (pad "1" thru_hole rect (at 0 0 90) (size 3 3) (drill 1.52) (layers "*.Cu" "*.Mask") (remove_unused_layers no) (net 3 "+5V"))
  (pad "2" thru_hole circle (at 5.08 0 90) (size 3 3) (drill 1.52) (layers "*.Cu" "*.Mask") (remove_unused_layers no) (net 11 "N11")))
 (gr_rect (start 123 53) (end 191 97) (stroke (width 0.05) (type default)) (fill none) (layer "Edge.Cuts"))
 (segment (start 175.405 60.595) (end 175.405 63.525) (width 0.2) (layer "F.Cu") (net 5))
 (segment (start 175.5 60.5) (end 175.405 60.595) (width 0.2) (layer "F.Cu") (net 5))
 (via (at 175.5 60.5) (size 0.6) (drill 0.3) (layers "F.Cu" "B.Cu") (free yes) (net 5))
 (segment (start 174.145 61.855) (end 175.5 60.5) (width 0.2) (layer "B.Cu") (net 5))
 (segment (start 136 90.58) (end 139.92 94.5) (width 0.2) (layer "B.Cu") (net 5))
 (segment (start 139.92 94.5) (end 150 94.5) (width 0.2) (layer "B.Cu") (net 5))
 (segment (start 159.4325 61.855) (end 174.145 61.855) (width 0.2) (layer "B.Cu") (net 5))
 (segment (start 155.2075 66.08) (end 155.2075 67.35) (width 0.2) (layer "B.Cu") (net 5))
 (segment (start 145 61.5) (end 150.6275 61.5) (width 0.2) (layer "B.Cu") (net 5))
 (segment (start 153.9375 68.62) (end 152.4 70.1575) (width 0.2) (layer "B.Cu") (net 5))
 (segment (start 155.2075 66.08) (end 159.4325 61.855) (width 0.2) (layer "B.Cu") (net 5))
 (segment (start 135.66 58) (end 141.5 58) (width 0.2) (layer "B.Cu") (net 5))
 (segment (start 150.96 93.54) (end 150.96 92) (width 0.2) (layer "B.Cu") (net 5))
 (segment (start 152.4 70.1575) (end 152.4 90.56) (width 0.2) (layer "B.Cu") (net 5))
 (segment (start 155.2075 67.35) (end 153.9375 68.62) (width 0.2) (layer "B.Cu") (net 5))
 (segment (start 152.4 90.56) (end 150.96 92) (width 0.2) (layer "B.Cu") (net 5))
 (segment (start 150 94.5) (end 150.96 93.54) (width 0.2) (layer "B.Cu") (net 5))
 (segment (start 150.6275 61.5) (end 155.2075 66.08) (width 0.2) (layer "B.Cu") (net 5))
 (segment (start 141.5 58) (end 145 61.5) (width 0.2) (layer "B.Cu") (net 5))
 (segment (start 179.5 70) (end 179.5 65.5) (width 0.2) (layer "F.Cu") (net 3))
 (segment (start 162.8275 66.08) (end 169.04 66.08) (width 0.2) (layer "F.Cu") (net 3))
 (segment (start 157.6775 72.5) (end 177 72.5) (width 0.2) (layer "F.Cu") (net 3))
 (segment (start 179.5 65.5) (end 187 58) (width 0.2) (layer "F.Cu") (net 3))
 (segment (start 161.5575 68.62) (end 157.6775 72.5) (width 0.2) (layer "F.Cu") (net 3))
 (segment (start 129.5 73) (end 127 70.5) (width 0.2) (layer "F.Cu") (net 3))
 (segment (start 139.76 76.76) (end 136 73) (width 0.2) (layer "F.Cu") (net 3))
 (segment (start 136 73) (end 129.5 73) (width 0.2) (layer "F.Cu") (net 3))
 (segment (start 143.34 76.76) (end 139.76 76.76) (width 0.2) (layer "F.Cu") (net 3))
 (segment (start 169.04 66.08) (end 171.595 63.525) (width 0.2) (layer "F.Cu") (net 3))
 (segment (start 162.8275 66.08) (end 162.8275 67.35) (width 0.2) (layer "F.Cu") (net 3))
 (segment (start 162.8275 67.35) (end 161.5575 68.62) (width 0.2) (layer "F.Cu") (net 3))
 (segment (start 143.34 76.76) (end 147.6 72.5) (width 0.2) (layer "F.Cu") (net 3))
 (segment (start 157.6775 72.5) (end 147.6 72.5) (width 0.2) (layer "F.Cu") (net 3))
 (segment (start 136.5 70.5) (end 136 70.5) (width 0.2) (layer "F.Cu") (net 3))
 (segment (start 177 72.5) (end 179.5 70) (width 0.2) (layer "F.Cu") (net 3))
 (segment (start 151 82.5) (end 154.5 82.5) (width 0.2) (layer "F.Cu") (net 12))
 (via (at 154.5 82.5) (size 0.6) (drill 0.3) (layers "F.Cu" "B.Cu") (free yes) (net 12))
 (via (at 151 82.5) (size 0.6) (drill 0.3) (layers "F.Cu" "B.Cu") (free yes) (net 12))
 (segment (start 125.5 58) (end 132 58) (width 0.2) (layer "B.Cu") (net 12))
 (segment (start 154.5 82.5) (end 154.5 87.92) (width 0.2) (layer "B.Cu") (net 12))
 (segment (start 134.5 60.5) (end 141.5 60.5) (width 0.2) (layer "B.Cu") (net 12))
 (segment (start 154.5 87.92) (end 158.58 92) (width 0.2) (layer "B.Cu") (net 12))
 (segment (start 132 58) (end 134.5 60.5) (width 0.2) (layer "B.Cu") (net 12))
 (segment (start 141.5 60.5) (end 145 64) (width 0.2) (layer "B.Cu") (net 12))
 (segment (start 149.52 81.02) (end 151 82.5) (width 0.2) (layer "B.Cu") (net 12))
 (segment (start 145 64) (end 145 64.04) (width 0.2) (layer "B.Cu") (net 12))
 (segment (start 149.52 68.56) (end 149.52 81.02) (width 0.2) (layer "B.Cu") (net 12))
 (segment (start 145 64.04) (end 149.52 68.56) (width 0.2) (layer "B.Cu") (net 12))
 (segment (start 130 84) (end 129.5 83.5) (width 0.2) (layer "F.Cu") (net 2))
 (segment (start 163.66 92) (end 155.66 84) (width 0.2) (layer "F.Cu") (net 2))
 (segment (start 136 84) (end 136 80.42) (width 0.2) (layer "F.Cu") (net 2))
 (segment (start 129.5 83.46) (end 127 80.96) (width 0.2) (layer "F.Cu") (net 2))
 (segment (start 155.66 84) (end 136 84) (width 0.2) (layer "F.Cu") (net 2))
 (segment (start 129.5 83.5) (end 129.5 83.46) (width 0.2) (layer "F.Cu") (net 2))
 (segment (start 136 84) (end 130 84) (width 0.2) (layer "F.Cu") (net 2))
 (segment (start 161.12 92) (end 155.16 86.04) (width 0.2) (layer "F.Cu") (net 1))
 (segment (start 155.16 86.04) (end 127 86.04) (width 0.2) (layer "F.Cu") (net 1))
 (segment (start 141.26 62.84) (end 145 66.58) (width 0.2) (layer "B.Cu") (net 11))
 (segment (start 127 65.42) (end 133.42 65.42) (width 0.2) (layer "B.Cu") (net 11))
 (segment (start 133.42 65.42) (end 136 62.84) (width 0.2) (layer "B.Cu") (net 11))
 (segment (start 136 62.84) (end 141.26 62.84) (width 0.2) (layer "B.Cu") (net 11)))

